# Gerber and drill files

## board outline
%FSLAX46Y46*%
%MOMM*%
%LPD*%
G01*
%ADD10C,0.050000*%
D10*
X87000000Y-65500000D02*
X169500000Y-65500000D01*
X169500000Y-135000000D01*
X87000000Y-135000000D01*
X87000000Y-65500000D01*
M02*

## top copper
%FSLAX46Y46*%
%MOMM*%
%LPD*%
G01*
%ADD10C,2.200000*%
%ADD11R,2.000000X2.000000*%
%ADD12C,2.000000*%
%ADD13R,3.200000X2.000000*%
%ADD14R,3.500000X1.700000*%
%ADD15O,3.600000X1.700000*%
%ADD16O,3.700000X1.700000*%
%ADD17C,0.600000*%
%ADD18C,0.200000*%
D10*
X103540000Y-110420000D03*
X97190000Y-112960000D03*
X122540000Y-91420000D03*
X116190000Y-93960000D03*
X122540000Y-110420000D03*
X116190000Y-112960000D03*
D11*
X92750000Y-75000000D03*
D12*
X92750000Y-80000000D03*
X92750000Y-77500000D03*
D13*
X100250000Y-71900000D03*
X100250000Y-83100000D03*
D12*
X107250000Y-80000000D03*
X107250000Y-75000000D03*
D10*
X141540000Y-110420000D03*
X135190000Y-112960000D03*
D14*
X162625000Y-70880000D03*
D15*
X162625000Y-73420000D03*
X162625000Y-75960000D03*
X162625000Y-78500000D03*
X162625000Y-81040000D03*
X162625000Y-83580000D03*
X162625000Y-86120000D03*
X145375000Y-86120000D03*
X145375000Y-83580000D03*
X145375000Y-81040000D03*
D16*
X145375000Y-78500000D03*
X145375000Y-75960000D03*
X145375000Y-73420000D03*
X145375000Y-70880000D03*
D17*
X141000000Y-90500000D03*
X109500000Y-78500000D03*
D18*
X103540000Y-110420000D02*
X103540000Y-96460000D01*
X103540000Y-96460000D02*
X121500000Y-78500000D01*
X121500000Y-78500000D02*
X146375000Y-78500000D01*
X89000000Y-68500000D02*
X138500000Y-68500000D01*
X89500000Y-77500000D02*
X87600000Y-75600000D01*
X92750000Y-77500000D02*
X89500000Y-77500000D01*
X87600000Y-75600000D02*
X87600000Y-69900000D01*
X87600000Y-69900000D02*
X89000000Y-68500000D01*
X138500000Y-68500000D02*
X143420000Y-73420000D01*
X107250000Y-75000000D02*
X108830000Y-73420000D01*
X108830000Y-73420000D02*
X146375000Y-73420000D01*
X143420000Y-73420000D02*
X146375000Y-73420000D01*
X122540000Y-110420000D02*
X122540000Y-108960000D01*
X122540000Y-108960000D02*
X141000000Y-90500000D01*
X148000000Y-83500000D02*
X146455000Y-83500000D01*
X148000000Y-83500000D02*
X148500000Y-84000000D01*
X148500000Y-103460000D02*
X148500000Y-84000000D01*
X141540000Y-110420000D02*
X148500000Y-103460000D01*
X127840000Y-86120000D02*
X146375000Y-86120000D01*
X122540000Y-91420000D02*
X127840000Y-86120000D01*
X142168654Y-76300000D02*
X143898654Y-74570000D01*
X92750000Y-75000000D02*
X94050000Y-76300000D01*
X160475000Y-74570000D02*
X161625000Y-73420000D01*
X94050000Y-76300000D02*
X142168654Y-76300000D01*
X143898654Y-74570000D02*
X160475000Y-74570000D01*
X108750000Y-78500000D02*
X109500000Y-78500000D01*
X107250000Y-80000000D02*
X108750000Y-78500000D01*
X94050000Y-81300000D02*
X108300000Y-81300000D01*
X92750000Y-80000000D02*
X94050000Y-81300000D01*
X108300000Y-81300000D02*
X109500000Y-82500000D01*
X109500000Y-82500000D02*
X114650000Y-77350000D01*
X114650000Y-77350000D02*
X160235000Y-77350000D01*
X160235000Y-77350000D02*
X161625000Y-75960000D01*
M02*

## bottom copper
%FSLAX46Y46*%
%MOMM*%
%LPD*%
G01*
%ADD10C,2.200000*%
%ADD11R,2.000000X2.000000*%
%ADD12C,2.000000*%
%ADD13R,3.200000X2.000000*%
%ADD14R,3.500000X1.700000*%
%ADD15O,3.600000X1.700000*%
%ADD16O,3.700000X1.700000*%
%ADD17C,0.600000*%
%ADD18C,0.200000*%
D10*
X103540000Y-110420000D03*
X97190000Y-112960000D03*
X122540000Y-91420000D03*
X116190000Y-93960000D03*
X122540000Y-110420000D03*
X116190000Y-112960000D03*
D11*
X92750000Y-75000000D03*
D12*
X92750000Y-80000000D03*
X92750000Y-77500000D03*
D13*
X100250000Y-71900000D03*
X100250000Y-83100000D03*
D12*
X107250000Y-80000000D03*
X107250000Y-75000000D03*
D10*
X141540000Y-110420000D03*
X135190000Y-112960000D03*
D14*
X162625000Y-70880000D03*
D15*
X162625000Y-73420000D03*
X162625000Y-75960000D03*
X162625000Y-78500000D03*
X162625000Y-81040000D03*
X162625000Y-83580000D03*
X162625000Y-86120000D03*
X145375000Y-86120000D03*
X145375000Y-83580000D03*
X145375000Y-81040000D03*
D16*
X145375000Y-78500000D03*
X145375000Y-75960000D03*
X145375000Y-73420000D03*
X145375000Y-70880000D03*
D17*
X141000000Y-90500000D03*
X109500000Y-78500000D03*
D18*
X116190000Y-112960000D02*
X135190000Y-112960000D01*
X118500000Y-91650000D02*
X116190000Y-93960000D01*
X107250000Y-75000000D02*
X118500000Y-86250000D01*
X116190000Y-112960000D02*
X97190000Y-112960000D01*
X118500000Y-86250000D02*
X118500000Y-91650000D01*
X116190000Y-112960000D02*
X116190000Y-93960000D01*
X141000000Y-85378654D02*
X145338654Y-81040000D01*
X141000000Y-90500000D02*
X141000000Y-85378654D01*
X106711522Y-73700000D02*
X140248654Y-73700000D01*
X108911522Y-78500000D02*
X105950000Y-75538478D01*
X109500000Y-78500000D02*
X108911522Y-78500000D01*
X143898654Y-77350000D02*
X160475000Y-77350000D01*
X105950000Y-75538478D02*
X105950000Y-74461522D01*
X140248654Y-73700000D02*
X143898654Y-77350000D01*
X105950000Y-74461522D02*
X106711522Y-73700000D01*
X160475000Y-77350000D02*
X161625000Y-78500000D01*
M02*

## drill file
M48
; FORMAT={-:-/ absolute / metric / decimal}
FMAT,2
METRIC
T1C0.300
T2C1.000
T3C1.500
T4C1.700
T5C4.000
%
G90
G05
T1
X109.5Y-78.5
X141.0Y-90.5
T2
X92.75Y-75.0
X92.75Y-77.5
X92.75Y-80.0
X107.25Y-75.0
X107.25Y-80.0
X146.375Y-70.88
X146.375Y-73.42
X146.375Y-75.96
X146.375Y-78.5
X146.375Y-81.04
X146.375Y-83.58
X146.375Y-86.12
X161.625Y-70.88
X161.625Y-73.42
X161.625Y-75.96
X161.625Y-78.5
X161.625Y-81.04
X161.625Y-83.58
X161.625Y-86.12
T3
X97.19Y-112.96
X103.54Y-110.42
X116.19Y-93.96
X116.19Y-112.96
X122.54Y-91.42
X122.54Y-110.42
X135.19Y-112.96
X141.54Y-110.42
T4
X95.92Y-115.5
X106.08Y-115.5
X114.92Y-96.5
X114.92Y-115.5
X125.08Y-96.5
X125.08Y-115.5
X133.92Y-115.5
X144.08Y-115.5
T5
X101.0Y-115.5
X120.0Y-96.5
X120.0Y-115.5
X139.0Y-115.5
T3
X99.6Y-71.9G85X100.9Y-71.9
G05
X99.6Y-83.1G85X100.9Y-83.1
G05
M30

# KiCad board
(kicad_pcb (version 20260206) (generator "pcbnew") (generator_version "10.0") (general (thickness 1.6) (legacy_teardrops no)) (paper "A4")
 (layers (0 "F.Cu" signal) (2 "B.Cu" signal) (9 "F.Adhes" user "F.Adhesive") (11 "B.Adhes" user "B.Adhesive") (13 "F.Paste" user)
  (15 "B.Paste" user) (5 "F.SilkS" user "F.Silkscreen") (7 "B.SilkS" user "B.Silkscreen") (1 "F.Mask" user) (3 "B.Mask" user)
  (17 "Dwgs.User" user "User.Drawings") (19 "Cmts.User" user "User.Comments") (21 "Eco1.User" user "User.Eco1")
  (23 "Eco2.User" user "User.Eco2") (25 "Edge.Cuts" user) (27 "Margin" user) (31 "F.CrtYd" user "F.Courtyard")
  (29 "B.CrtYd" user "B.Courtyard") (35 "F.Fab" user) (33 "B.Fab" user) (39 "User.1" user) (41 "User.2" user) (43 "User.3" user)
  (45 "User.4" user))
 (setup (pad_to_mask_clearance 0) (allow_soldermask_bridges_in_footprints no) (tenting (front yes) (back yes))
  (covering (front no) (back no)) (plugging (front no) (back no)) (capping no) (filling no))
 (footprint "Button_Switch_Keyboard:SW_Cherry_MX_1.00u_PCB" (layer "F.Cu") (at 103.54 110.42)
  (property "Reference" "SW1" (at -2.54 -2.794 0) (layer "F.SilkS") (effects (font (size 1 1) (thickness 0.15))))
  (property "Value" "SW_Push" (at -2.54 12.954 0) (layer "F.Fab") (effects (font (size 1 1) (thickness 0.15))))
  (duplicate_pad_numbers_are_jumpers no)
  (pad "" np_thru_hole circle (at -7.62 5.08) (size 1.7 1.7) (drill 1.7) (layers "*.Cu" "*.Mask"))
  (pad "" np_thru_hole circle (at -2.54 5.08) (size 4 4) (drill 4) (layers "*.Cu" "*.Mask"))
  (pad "" np_thru_hole circle (at 2.54 5.08) (size 1.7 1.7) (drill 1.7) (layers "*.Cu" "*.Mask"))
  (pad "1" thru_hole circle (at 0 0) (size 2.2 2.2) (drill 1.5) (layers "*.Cu" "*.Mask") (remove_unused_layers no)
   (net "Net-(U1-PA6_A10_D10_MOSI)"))
  (pad "2" thru_hole circle (at -6.35 2.54) (size 2.2 2.2) (drill 1.5) (layers "*.Cu" "*.Mask") (remove_unused_layers no) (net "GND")))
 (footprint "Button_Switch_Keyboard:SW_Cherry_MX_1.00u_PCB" (layer "F.Cu") (at 122.54 91.42)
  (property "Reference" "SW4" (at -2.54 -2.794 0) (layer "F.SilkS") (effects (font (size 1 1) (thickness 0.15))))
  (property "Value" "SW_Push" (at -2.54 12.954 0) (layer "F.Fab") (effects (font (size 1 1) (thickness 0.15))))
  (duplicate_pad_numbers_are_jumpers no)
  (pad "" np_thru_hole circle (at -7.62 5.08) (size 1.7 1.7) (drill 1.7) (layers "*.Cu" "*.Mask"))
  (pad "" np_thru_hole circle (at -2.54 5.08) (size 4 4) (drill 4) (layers "*.Cu" "*.Mask"))
  (pad "" np_thru_hole circle (at 2.54 5.08) (size 1.7 1.7) (drill 1.7) (layers "*.Cu" "*.Mask"))
  (pad "1" thru_hole circle (at 0 0) (size 2.2 2.2) (drill 1.5) (layers "*.Cu" "*.Mask") (remove_unused_layers no)
   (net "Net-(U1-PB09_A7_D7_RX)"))
  (pad "2" thru_hole circle (at -6.35 2.54) (size 2.2 2.2) (drill 1.5) (layers "*.Cu" "*.Mask") (remove_unused_layers no) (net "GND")))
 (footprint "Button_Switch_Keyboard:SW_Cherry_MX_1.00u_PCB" (layer "F.Cu") (at 122.54 110.42)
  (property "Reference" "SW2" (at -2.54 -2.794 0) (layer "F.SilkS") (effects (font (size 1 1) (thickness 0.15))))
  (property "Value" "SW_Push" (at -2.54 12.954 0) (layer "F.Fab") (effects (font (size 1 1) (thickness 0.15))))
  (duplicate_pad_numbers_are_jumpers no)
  (pad "" np_thru_hole circle (at -7.62 5.08) (size 1.7 1.7) (drill 1.7) (layers "*.Cu" "*.Mask"))
  (pad "" np_thru_hole circle (at -2.54 5.08) (size 4 4) (drill 4) (layers "*.Cu" "*.Mask"))
  (pad "" np_thru_hole circle (at 2.54 5.08) (size 1.7 1.7) (drill 1.7) (layers "*.Cu" "*.Mask"))
  (pad "1" thru_hole circle (at 0 0) (size 2.2 2.2) (drill 1.5) (layers "*.Cu" "*.Mask") (remove_unused_layers no)
   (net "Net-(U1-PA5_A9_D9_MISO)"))
  (pad "2" thru_hole circle (at -6.35 2.54) (size 2.2 2.2) (drill 1.5) (layers "*.Cu" "*.Mask") (remove_unused_layers no) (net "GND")))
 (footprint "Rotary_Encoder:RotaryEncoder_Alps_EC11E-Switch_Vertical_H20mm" (layer "F.Cu") (at 92.75 75)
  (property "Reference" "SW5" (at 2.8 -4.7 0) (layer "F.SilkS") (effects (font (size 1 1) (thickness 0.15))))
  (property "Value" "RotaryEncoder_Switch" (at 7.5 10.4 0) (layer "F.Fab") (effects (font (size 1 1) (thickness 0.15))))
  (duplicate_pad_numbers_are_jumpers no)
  (pad "A" thru_hole rect (at 0 0) (size 2 2) (drill 1) (layers "*.Cu" "*.Mask") (remove_unused_layers no) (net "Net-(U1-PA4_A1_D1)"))
  (pad "B" thru_hole circle (at 0 5) (size 2 2) (drill 1) (layers "*.Cu" "*.Mask") (remove_unused_layers no) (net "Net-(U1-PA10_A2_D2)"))
  (pad "C" thru_hole circle (at 0 2.5) (size 2 2) (drill 1) (layers "*.Cu" "*.Mask") (remove_unused_layers no) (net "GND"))
  (pad "MP" thru_hole rect (at 7.5 -3.1) (size 3.2 2) (drill oval 2.8 1.5) (layers "*.Cu" "*.Mask") (remove_unused_layers no))
  (pad "MP" thru_hole rect (at 7.5 8.1) (size 3.2 2) (drill oval 2.8 1.5) (layers "*.Cu" "*.Mask") (remove_unused_layers no))
  (pad "S1" thru_hole circle (at 14.5 5) (size 2 2) (drill 1) (layers "*.Cu" "*.Mask") (remove_unused_layers no) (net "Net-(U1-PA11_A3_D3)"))
  (pad "S2" thru_hole circle (at 14.5 0) (size 2 2) (drill 1) (layers "*.Cu" "*.Mask") (remove_unused_layers no) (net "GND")))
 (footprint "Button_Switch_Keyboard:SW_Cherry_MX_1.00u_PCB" (layer "F.Cu") (at 141.54 110.42)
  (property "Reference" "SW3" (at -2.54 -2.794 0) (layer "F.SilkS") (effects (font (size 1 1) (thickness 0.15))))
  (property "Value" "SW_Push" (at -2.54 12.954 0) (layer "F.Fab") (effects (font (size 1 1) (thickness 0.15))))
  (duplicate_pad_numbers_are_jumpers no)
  (pad "" np_thru_hole circle (at -7.62 5.08) (size 1.7 1.7) (drill 1.7) (layers "*.Cu" "*.Mask"))
  (pad "" np_thru_hole circle (at -2.54 5.08) (size 4 4) (drill 4) (layers "*.Cu" "*.Mask"))
  (pad "" np_thru_hole circle (at 2.54 5.08) (size 1.7 1.7) (drill 1.7) (layers "*.Cu" "*.Mask"))
  (pad "1" thru_hole circle (at 0 0) (size 2.2 2.2) (drill 1.5) (layers "*.Cu" "*.Mask") (remove_unused_layers no)
   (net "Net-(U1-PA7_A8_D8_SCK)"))
  (pad "2" thru_hole circle (at -6.35 2.54) (size 2.2 2.2) (drill 1.5) (layers "*.Cu" "*.Mask") (remove_unused_layers no) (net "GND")))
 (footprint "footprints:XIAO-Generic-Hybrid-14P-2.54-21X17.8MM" (layer "B.Cu") (at 154 78.5 180)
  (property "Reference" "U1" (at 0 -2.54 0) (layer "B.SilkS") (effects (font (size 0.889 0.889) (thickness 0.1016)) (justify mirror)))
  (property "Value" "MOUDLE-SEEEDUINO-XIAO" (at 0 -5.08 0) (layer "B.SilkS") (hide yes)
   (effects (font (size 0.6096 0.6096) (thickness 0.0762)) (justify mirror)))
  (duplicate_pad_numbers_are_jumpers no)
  (pad "1" thru_hole rect (at -7.625 7.62 180) (size 3.5 1.7) (drill 1 (offset -1 0)) (layers "*.Cu" "*.Mask") (remove_unused_layers no)
   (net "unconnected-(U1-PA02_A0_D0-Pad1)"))
  (pad "2" thru_hole oval (at -7.625 5.08 180) (size 3.6 1.7) (drill 1 (offset -1 0)) (layers "*.Cu" "*.Mask") (remove_unused_layers no)
   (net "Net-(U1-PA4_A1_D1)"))
  (pad "3" thru_hole oval (at -7.625 2.54 180) (size 3.6 1.7) (drill 1 (offset -1 0)) (layers "*.Cu" "*.Mask") (remove_unused_layers no)
   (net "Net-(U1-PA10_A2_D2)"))
  (pad "4" thru_hole oval (at -7.625 0 180) (size 3.6 1.7) (drill 1 (offset -1 0)) (layers "*.Cu" "*.Mask") (remove_unused_layers no)
   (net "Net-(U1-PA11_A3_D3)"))
  (pad "5" thru_hole oval (at -7.625 -2.54 180) (size 3.6 1.7) (drill 1 (offset -1 0)) (layers "*.Cu" "*.Mask") (remove_unused_layers no)
   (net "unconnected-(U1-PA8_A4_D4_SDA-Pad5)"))
  (pad "6" thru_hole oval (at -7.625 -5.08) (size 3.6 1.7) (drill 1 (offset 1 0)) (layers "*.Cu" "*.Mask") (remove_unused_layers no)
   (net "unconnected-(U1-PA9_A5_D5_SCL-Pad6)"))
  (pad "7" thru_hole oval (at -7.625 -7.62 180) (size 3.6 1.7) (drill 1 (offset -1 0)) (layers "*.Cu" "*.Mask") (remove_unused_layers no)
   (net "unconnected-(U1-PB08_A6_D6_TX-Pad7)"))
  (pad "8" thru_hole oval (at 7.625 -7.62 180) (size 3.6 1.7) (drill 1 (offset 1 0)) (layers "*.Cu" "*.Mask") (remove_unused_layers no)
   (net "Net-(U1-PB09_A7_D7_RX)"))
  (pad "9" thru_hole oval (at 7.625 -5.08 180) (size 3.6 1.7) (drill 1 (offset 1 0)) (layers "*.Cu" "*.Mask") (remove_unused_layers no)
   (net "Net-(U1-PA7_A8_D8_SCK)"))
  (pad "10" thru_hole oval (at 7.625 -2.54 180) (size 3.6 1.7) (drill 1 (offset 1 0)) (layers "*.Cu" "*.Mask") (remove_unused_layers no)
   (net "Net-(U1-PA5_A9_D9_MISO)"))
  (pad "11" thru_hole oval (at 7.625 0 180) (size 3.7 1.7) (drill 1 (offset 1 0)) (layers "*.Cu" "*.Mask") (remove_unused_layers no)
   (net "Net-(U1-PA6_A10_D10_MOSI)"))
  (pad "12" thru_hole oval (at 7.625 2.54 180) (size 3.7 1.7) (drill 1 (offset 1 0)) (layers "*.Cu" "*.Mask") (remove_unused_layers no)
   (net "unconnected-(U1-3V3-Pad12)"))
  (pad "13" thru_hole oval (at 7.625 5.08 180) (size 3.7 1.7) (drill 1 (offset 1 0)) (layers "*.Cu" "*.Mask") (remove_unused_layers no)
   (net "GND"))
  (pad "14" thru_hole oval (at 7.625 7.62 180) (size 3.7 1.7) (drill 1 (offset 1 0)) (layers "*.Cu" "*.Mask") (remove_unused_layers no)
   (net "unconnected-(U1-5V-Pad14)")))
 (gr_rect (start 87 65.5) (end 169.5 135) (stroke (width 0.05) (type solid)) (fill no) (layer "Edge.Cuts"))
 (segment (start 103.54 110.42) (end 103.54 96.46) (width 0.2) (layer "F.Cu") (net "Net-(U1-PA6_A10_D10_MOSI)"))
 (segment (start 103.54 96.46) (end 121.5 78.5) (width 0.2) (layer "F.Cu") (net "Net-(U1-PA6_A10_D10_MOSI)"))
 (segment (start 121.5 78.5) (end 146.375 78.5) (width 0.2) (layer "F.Cu") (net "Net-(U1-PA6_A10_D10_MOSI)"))
 (segment (start 89 68.5) (end 138.5 68.5) (width 0.2) (layer "F.Cu") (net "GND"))
 (segment (start 89.5 77.5) (end 87.6 75.6) (width 0.2) (layer "F.Cu") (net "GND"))
 (segment (start 92.75 77.5) (end 89.5 77.5) (width 0.2) (layer "F.Cu") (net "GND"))
 (segment (start 87.6 75.6) (end 87.6 69.9) (width 0.2) (layer "F.Cu") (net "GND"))
 (segment (start 87.6 69.9) (end 89 68.5) (width 0.2) (layer "F.Cu") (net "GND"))
 (segment (start 138.5 68.5) (end 143.42 73.42) (width 0.2) (layer "F.Cu") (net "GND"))
 (segment (start 107.25 75) (end 108.83 73.42) (width 0.2) (layer "F.Cu") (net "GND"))
 (segment (start 108.83 73.42) (end 146.375 73.42) (width 0.2) (layer "F.Cu") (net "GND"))
 (segment (start 143.42 73.42) (end 146.375 73.42) (width 0.2) (layer "F.Cu") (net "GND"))
 (segment (start 116.19 112.96) (end 135.19 112.96) (width 0.2) (layer "B.Cu") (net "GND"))
 (segment (start 118.5 91.65) (end 116.19 93.96) (width 0.2) (layer "B.Cu") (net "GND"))
 (segment (start 107.25 75) (end 118.5 86.25) (width 0.2) (layer "B.Cu") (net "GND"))
 (segment (start 116.19 112.96) (end 97.19 112.96) (width 0.2) (layer "B.Cu") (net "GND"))
 (segment (start 118.5 86.25) (end 118.5 91.65) (width 0.2) (layer "B.Cu") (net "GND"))
 (segment (start 116.19 112.96) (end 116.19 93.96) (width 0.2) (layer "B.Cu") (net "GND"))
 (segment (start 122.54 110.42) (end 122.54 108.96) (width 0.2) (layer "F.Cu") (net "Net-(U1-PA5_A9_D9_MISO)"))
 (segment (start 122.54 108.96) (end 141 90.5) (width 0.2) (layer "F.Cu") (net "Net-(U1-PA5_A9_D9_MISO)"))
 (via (at 141 90.5) (size 0.6) (drill 0.3) (layers "F.Cu" "B.Cu") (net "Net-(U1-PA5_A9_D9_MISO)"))
 (segment (start 141 85.378654) (end 145.338654 81.04) (width 0.2) (layer "B.Cu") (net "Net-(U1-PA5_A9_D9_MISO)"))
 (segment (start 141 90.5) (end 141 85.378654) (width 0.2) (layer "B.Cu") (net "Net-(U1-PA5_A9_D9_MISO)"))
 (segment (start 148 83.5) (end 146.455 83.5) (width 0.2) (layer "F.Cu") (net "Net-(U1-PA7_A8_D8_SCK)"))
 (segment (start 148 83.5) (end 148.5 84) (width 0.2) (layer "F.Cu") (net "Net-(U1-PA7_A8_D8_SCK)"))
 (segment (start 148.5 103.46) (end 148.5 84) (width 0.2) (layer "F.Cu") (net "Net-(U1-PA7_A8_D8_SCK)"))
 (segment (start 141.54 110.42) (end 148.5 103.46) (width 0.2) (layer "F.Cu") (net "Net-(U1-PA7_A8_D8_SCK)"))
 (segment (start 127.84 86.12) (end 146.375 86.12) (width 0.2) (layer "F.Cu") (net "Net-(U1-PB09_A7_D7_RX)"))
 (segment (start 122.54 91.42) (end 127.84 86.12) (width 0.2) (layer "F.Cu") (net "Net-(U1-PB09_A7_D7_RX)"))
 (segment (start 142.168654 76.3) (end 143.898654 74.57) (width 0.2) (layer "F.Cu") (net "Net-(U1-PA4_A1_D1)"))
 (segment (start 92.75 75) (end 94.05 76.3) (width 0.2) (layer "F.Cu") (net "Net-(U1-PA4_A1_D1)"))
 (segment (start 160.475 74.57) (end 161.625 73.42) (width 0.2) (layer "F.Cu") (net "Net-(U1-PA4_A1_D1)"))
 (segment (start 94.05 76.3) (end 142.168654 76.3) (width 0.2) (layer "F.Cu") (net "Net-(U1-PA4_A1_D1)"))
 (segment (start 143.898654 74.57) (end 160.475 74.57) (width 0.2) (layer "F.Cu") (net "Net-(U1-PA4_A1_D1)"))
 (segment (start 108.75 78.5) (end 109.5 78.5) (width 0.2) (layer "F.Cu") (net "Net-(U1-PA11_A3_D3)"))
 (segment (start 107.25 80) (end 108.75 78.5) (width 0.2) (layer "F.Cu") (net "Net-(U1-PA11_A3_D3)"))
 (via (at 109.5 78.5) (size 0.6) (drill 0.3) (layers "F.Cu" "B.Cu") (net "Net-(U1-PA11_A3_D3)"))
 (segment (start 106.711522 73.7) (end 140.248654 73.7) (width 0.2) (layer "B.Cu") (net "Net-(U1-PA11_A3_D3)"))
 (segment (start 108.911522 78.5) (end 105.95 75.538478) (width 0.2) (layer "B.Cu") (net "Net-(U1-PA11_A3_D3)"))
 (segment (start 109.5 78.5) (end 108.911522 78.5) (width 0.2) (layer "B.Cu") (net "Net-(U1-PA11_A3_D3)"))
 (segment (start 143.898654 77.35) (end 160.475 77.35) (width 0.2) (layer "B.Cu") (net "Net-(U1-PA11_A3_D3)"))
 (segment (start 105.95 75.538478) (end 105.95 74.461522) (width 0.2) (layer "B.Cu") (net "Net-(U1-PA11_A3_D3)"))
 (segment (start 140.248654 73.7) (end 143.898654 77.35) (width 0.2) (layer "B.Cu") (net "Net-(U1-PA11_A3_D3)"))
 (segment (start 105.95 74.461522) (end 106.711522 73.7) (width 0.2) (layer "B.Cu") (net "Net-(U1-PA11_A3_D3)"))
 (segment (start 160.475 77.35) (end 161.625 78.5) (width 0.2) (layer "B.Cu") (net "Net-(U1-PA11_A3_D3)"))
 (segment (start 94.05 81.3) (end 108.3 81.3) (width 0.2) (layer "F.Cu") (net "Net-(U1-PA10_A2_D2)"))
 (segment (start 92.75 80) (end 94.05 81.3) (width 0.2) (layer "F.Cu") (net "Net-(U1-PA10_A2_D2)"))
 (segment (start 108.3 81.3) (end 109.5 82.5) (width 0.2) (layer "F.Cu") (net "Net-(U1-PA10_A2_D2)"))
 (segment (start 109.5 82.5) (end 114.65 77.35) (width 0.2) (layer "F.Cu") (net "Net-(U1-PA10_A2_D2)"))
 (segment (start 114.65 77.35) (end 160.235 77.35) (width 0.2) (layer "F.Cu") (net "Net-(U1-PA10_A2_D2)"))
 (segment (start 160.235 77.35) (end 161.625 75.96) (width 0.2) (layer "F.Cu") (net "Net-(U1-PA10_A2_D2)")))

